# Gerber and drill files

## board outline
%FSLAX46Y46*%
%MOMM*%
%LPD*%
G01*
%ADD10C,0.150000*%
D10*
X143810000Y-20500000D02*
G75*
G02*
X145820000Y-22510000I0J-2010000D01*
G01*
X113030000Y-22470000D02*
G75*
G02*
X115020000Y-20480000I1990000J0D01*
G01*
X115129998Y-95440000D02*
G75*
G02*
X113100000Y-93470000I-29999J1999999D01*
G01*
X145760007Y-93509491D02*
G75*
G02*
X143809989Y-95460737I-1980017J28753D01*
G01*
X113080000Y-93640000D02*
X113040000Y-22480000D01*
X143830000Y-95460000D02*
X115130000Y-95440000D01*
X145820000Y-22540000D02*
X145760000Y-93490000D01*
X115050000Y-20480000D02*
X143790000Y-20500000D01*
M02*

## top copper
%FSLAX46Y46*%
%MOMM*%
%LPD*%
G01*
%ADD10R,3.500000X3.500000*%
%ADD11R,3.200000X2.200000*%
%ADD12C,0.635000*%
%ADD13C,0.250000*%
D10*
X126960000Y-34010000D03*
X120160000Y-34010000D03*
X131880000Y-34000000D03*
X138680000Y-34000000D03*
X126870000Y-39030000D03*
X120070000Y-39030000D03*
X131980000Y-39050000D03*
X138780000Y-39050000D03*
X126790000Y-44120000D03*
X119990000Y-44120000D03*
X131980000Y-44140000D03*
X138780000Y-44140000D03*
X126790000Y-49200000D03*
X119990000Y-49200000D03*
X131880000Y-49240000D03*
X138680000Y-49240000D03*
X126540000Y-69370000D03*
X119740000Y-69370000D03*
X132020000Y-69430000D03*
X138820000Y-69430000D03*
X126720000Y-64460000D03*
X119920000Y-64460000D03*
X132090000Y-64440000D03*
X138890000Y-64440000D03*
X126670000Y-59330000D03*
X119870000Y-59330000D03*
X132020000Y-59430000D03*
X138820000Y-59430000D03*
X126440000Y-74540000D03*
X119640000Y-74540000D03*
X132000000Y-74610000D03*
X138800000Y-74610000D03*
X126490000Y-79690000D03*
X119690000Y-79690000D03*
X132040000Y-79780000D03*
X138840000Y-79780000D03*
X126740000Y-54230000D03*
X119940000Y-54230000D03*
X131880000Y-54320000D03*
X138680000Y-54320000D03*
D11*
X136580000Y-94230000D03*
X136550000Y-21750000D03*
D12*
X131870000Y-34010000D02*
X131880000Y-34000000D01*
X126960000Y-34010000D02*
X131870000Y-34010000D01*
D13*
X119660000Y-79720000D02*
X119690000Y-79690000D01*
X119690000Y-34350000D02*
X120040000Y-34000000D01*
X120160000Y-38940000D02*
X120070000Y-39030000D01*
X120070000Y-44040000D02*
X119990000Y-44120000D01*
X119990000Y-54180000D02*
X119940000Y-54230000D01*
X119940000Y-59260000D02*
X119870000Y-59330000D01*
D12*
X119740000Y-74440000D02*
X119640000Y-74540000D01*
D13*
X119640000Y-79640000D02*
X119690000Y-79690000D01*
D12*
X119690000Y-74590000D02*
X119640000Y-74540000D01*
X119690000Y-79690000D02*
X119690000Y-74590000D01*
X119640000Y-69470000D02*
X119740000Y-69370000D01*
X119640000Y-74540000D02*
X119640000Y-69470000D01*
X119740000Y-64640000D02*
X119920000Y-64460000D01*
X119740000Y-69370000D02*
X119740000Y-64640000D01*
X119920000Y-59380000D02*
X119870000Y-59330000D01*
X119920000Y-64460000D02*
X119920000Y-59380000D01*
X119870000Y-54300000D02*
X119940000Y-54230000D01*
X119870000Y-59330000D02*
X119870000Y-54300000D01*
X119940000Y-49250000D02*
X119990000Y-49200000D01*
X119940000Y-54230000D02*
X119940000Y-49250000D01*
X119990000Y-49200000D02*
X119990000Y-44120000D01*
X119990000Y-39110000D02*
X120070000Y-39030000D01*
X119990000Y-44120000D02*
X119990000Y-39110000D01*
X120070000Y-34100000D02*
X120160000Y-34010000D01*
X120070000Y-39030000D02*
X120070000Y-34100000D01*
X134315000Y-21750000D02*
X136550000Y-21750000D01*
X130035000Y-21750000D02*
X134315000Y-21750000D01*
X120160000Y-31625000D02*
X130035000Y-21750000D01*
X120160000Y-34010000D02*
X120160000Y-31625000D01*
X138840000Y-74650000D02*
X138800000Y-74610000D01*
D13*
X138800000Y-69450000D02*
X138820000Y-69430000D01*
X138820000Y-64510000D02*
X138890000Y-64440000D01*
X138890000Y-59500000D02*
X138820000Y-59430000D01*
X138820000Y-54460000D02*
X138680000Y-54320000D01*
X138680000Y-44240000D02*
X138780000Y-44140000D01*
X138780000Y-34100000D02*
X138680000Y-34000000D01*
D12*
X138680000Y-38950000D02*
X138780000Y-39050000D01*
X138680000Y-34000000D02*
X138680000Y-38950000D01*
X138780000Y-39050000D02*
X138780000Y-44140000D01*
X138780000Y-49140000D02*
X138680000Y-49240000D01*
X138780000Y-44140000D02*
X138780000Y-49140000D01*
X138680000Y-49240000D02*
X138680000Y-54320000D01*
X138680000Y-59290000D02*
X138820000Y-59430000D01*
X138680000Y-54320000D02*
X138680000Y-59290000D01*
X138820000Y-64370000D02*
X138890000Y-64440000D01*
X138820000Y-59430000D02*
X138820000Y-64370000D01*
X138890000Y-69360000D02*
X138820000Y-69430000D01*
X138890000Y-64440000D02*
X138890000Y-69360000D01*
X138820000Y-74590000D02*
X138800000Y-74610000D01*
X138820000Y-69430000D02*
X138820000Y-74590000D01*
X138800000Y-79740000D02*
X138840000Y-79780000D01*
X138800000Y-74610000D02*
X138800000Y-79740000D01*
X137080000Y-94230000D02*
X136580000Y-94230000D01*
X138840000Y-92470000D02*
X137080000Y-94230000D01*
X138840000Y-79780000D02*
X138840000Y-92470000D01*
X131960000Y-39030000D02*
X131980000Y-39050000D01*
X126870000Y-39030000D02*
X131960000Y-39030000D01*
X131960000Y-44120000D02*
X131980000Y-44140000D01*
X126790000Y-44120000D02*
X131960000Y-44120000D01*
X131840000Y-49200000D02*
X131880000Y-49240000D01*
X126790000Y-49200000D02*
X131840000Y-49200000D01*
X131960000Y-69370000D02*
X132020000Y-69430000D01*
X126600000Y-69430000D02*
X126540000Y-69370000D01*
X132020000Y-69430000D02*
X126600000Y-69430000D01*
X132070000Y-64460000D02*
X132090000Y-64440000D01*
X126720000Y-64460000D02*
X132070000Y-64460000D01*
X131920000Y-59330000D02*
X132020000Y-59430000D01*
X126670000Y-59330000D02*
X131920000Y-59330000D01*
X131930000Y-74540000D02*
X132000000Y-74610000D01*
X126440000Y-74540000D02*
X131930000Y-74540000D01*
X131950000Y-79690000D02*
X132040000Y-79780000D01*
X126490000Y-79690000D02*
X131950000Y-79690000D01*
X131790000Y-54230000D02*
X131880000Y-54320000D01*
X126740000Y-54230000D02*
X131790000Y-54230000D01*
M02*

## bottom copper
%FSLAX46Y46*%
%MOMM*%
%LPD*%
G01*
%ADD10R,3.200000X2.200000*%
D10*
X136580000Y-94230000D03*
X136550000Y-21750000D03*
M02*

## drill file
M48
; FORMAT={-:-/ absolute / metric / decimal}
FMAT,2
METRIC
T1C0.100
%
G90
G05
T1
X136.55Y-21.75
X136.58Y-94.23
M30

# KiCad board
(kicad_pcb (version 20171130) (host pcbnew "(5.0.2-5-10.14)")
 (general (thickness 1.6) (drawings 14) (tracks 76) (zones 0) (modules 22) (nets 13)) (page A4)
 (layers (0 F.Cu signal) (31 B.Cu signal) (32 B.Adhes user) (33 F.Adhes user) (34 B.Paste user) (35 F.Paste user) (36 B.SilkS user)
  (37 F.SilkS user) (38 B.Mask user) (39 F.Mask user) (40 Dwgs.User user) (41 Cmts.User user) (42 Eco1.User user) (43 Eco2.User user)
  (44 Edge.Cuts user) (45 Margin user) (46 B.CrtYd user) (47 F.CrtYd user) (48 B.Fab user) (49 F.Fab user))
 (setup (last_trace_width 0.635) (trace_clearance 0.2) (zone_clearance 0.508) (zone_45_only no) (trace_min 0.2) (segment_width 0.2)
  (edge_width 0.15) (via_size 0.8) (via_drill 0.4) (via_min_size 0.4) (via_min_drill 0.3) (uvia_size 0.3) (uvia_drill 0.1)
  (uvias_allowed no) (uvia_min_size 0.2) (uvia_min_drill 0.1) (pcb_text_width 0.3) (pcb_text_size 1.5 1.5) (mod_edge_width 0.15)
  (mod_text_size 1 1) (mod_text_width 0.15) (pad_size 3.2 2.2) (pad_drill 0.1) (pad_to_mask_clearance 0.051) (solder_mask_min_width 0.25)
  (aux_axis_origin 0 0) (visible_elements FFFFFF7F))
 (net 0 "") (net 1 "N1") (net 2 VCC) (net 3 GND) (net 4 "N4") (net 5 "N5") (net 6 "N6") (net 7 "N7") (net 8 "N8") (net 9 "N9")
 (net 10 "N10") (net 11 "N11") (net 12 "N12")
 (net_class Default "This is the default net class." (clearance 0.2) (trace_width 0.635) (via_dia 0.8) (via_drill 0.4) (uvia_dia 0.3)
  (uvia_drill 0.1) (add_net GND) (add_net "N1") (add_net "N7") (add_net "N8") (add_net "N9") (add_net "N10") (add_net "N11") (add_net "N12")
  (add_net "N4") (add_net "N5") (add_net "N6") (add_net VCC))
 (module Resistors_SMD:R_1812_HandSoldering (layer F.Cu) (at 123.56 34.01)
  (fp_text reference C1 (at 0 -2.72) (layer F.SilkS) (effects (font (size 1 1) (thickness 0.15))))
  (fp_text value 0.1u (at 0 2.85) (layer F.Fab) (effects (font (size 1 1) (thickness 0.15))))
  (pad 2 smd rect (at 3.4 0) (size 3.5 3.5) (layers F.Cu F.Paste F.Mask) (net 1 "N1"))
  (pad 1 smd rect (at -3.4 0) (size 3.5 3.5) (layers F.Cu F.Paste F.Mask) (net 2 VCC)))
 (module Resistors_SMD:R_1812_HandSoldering (layer F.Cu) (at 135.28 34)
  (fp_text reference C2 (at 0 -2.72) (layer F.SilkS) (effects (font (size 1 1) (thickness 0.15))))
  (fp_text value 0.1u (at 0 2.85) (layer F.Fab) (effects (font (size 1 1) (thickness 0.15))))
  (pad 1 smd rect (at -3.4 0) (size 3.5 3.5) (layers F.Cu F.Paste F.Mask) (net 1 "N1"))
  (pad 2 smd rect (at 3.4 0) (size 3.5 3.5) (layers F.Cu F.Paste F.Mask) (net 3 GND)))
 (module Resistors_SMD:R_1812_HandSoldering (layer F.Cu) (at 123.47 39.03)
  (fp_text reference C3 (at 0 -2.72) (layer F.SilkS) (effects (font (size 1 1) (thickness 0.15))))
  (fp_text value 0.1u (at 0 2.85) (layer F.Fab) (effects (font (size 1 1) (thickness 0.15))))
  (pad 2 smd rect (at 3.4 0) (size 3.5 3.5) (layers F.Cu F.Paste F.Mask) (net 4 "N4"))
  (pad 1 smd rect (at -3.4 0) (size 3.5 3.5) (layers F.Cu F.Paste F.Mask) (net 2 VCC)))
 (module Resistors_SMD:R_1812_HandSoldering (layer F.Cu) (at 135.38 39.05)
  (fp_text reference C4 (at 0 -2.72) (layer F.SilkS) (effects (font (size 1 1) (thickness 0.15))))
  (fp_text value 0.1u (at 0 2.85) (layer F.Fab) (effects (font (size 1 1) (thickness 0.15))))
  (pad 1 smd rect (at -3.4 0) (size 3.5 3.5) (layers F.Cu F.Paste F.Mask) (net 4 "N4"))
  (pad 2 smd rect (at 3.4 0) (size 3.5 3.5) (layers F.Cu F.Paste F.Mask) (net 3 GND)))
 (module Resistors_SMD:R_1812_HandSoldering (layer F.Cu) (at 123.39 44.12)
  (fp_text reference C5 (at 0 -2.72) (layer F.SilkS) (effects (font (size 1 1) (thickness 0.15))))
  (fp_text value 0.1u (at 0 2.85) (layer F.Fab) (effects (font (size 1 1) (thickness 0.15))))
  (pad 2 smd rect (at 3.4 0) (size 3.5 3.5) (layers F.Cu F.Paste F.Mask) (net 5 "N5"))
  (pad 1 smd rect (at -3.4 0) (size 3.5 3.5) (layers F.Cu F.Paste F.Mask) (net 2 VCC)))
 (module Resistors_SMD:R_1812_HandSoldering (layer F.Cu) (at 135.38 44.14)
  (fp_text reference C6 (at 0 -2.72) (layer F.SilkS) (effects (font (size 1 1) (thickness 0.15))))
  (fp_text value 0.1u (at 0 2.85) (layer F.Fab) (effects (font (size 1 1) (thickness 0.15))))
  (pad 1 smd rect (at -3.4 0) (size 3.5 3.5) (layers F.Cu F.Paste F.Mask) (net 5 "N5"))
  (pad 2 smd rect (at 3.4 0) (size 3.5 3.5) (layers F.Cu F.Paste F.Mask) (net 3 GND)))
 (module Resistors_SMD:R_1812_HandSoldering (layer F.Cu) (at 123.39 49.2)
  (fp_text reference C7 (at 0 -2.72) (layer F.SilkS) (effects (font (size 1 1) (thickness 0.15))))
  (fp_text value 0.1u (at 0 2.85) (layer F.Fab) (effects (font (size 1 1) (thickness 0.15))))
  (pad 2 smd rect (at 3.4 0) (size 3.5 3.5) (layers F.Cu F.Paste F.Mask) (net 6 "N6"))
  (pad 1 smd rect (at -3.4 0) (size 3.5 3.5) (layers F.Cu F.Paste F.Mask) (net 2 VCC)))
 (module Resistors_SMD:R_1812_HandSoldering (layer F.Cu) (at 135.28 49.24)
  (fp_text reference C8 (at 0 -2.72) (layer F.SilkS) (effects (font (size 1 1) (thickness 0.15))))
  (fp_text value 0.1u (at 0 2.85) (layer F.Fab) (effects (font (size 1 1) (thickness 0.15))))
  (pad 1 smd rect (at -3.4 0) (size 3.5 3.5) (layers F.Cu F.Paste F.Mask) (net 6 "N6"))
  (pad 2 smd rect (at 3.4 0) (size 3.5 3.5) (layers F.Cu F.Paste F.Mask) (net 3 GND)))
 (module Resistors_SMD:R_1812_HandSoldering (layer F.Cu) (at 123.14 69.37)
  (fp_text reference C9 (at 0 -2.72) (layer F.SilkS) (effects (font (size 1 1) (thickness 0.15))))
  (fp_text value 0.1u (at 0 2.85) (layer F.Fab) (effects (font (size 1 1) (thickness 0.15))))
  (pad 2 smd rect (at 3.4 0) (size 3.5 3.5) (layers F.Cu F.Paste F.Mask) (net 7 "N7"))
  (pad 1 smd rect (at -3.4 0) (size 3.5 3.5) (layers F.Cu F.Paste F.Mask) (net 2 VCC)))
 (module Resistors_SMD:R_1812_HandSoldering (layer F.Cu) (at 135.42 69.43)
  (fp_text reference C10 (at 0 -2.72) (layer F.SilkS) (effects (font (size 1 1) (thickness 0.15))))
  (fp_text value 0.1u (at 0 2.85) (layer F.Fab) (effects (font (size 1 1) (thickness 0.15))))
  (pad 1 smd rect (at -3.4 0) (size 3.5 3.5) (layers F.Cu F.Paste F.Mask) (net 7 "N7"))
  (pad 2 smd rect (at 3.4 0) (size 3.5 3.5) (layers F.Cu F.Paste F.Mask) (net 3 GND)))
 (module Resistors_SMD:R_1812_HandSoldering (layer F.Cu) (at 123.32 64.46)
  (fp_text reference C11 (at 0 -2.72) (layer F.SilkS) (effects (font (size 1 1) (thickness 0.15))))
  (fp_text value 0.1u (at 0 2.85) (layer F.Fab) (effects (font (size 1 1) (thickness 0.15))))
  (pad 2 smd rect (at 3.4 0) (size 3.5 3.5) (layers F.Cu F.Paste F.Mask) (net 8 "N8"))
  (pad 1 smd rect (at -3.4 0) (size 3.5 3.5) (layers F.Cu F.Paste F.Mask) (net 2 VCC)))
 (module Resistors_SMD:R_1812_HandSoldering (layer F.Cu) (at 135.49 64.44)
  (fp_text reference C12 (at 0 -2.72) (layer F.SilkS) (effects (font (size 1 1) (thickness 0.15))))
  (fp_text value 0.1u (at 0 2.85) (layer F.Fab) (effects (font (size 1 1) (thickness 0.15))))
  (pad 1 smd rect (at -3.4 0) (size 3.5 3.5) (layers F.Cu F.Paste F.Mask) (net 8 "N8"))
  (pad 2 smd rect (at 3.4 0) (size 3.5 3.5) (layers F.Cu F.Paste F.Mask) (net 3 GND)))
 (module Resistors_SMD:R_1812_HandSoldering (layer F.Cu) (at 123.27 59.33)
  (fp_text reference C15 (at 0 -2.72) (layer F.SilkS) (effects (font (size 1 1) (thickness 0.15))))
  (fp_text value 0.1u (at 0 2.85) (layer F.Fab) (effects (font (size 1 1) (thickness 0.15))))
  (pad 2 smd rect (at 3.4 0) (size 3.5 3.5) (layers F.Cu F.Paste F.Mask) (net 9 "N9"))
  (pad 1 smd rect (at -3.4 0) (size 3.5 3.5) (layers F.Cu F.Paste F.Mask) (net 2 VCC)))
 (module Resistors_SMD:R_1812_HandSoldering (layer F.Cu) (at 135.42 59.43)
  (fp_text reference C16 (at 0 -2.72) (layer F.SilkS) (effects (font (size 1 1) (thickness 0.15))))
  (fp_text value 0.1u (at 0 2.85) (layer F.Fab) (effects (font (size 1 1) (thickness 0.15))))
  (pad 1 smd rect (at -3.4 0) (size 3.5 3.5) (layers F.Cu F.Paste F.Mask) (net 9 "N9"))
  (pad 2 smd rect (at 3.4 0) (size 3.5 3.5) (layers F.Cu F.Paste F.Mask) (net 3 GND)))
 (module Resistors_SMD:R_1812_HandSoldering (layer F.Cu) (at 123.04 74.54)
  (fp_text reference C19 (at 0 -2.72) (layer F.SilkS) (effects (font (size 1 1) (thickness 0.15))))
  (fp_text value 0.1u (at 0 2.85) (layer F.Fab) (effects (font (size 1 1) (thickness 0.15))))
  (pad 2 smd rect (at 3.4 0) (size 3.5 3.5) (layers F.Cu F.Paste F.Mask) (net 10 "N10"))
  (pad 1 smd rect (at -3.4 0) (size 3.5 3.5) (layers F.Cu F.Paste F.Mask) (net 2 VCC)))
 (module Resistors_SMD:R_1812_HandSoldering (layer F.Cu) (at 135.4 74.61)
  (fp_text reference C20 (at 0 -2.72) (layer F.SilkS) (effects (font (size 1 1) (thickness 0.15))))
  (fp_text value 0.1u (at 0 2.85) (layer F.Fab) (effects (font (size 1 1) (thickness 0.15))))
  (pad 1 smd rect (at -3.4 0) (size 3.5 3.5) (layers F.Cu F.Paste F.Mask) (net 10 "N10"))
  (pad 2 smd rect (at 3.4 0) (size 3.5 3.5) (layers F.Cu F.Paste F.Mask) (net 3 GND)))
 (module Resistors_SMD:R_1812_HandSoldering (layer F.Cu) (at 123.09 79.69)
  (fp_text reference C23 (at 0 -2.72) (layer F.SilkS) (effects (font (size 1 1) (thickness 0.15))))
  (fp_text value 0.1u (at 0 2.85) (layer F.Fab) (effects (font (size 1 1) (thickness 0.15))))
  (pad 2 smd rect (at 3.4 0) (size 3.5 3.5) (layers F.Cu F.Paste F.Mask) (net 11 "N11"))
  (pad 1 smd rect (at -3.4 0) (size 3.5 3.5) (layers F.Cu F.Paste F.Mask) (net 2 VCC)))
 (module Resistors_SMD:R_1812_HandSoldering (layer F.Cu) (at 135.44 79.78)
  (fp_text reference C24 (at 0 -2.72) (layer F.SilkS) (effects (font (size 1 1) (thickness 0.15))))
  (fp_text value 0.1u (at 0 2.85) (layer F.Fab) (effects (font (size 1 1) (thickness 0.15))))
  (pad 1 smd rect (at -3.4 0) (size 3.5 3.5) (layers F.Cu F.Paste F.Mask) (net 11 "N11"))
  (pad 2 smd rect (at 3.4 0) (size 3.5 3.5) (layers F.Cu F.Paste F.Mask) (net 3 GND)))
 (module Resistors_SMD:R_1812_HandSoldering (layer F.Cu) (at 123.34 54.23)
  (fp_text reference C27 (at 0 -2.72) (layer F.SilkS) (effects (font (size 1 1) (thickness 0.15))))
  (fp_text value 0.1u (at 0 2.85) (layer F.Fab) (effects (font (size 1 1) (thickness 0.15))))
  (pad 2 smd rect (at 3.4 0) (size 3.5 3.5) (layers F.Cu F.Paste F.Mask) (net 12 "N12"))
  (pad 1 smd rect (at -3.4 0) (size 3.5 3.5) (layers F.Cu F.Paste F.Mask) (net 2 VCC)))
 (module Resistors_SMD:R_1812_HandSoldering (layer F.Cu) (at 135.28 54.32)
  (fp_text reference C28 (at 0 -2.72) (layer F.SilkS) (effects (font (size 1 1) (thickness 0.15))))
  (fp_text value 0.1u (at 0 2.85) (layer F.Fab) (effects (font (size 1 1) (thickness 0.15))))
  (pad 1 smd rect (at -3.4 0) (size 3.5 3.5) (layers F.Cu F.Paste F.Mask) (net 12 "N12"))
  (pad 2 smd rect (at 3.4 0) (size 3.5 3.5) (layers F.Cu F.Paste F.Mask) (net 3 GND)))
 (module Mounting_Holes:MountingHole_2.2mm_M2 (layer F.Cu) (at 136.58 94.23)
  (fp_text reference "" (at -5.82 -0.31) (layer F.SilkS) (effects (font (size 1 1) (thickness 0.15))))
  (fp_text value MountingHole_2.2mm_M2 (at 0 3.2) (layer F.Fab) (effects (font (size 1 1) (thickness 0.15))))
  (pad "" thru_hole rect (at 0 0) (size 3.2 2.2) (drill 0.1) (layers *.Cu *.Mask) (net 3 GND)))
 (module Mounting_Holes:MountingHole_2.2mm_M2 (layer F.Cu) (at 136.55 21.75)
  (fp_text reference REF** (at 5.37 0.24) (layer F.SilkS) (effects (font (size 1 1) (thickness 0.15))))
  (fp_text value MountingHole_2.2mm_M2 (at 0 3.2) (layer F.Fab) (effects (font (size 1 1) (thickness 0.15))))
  (pad "" thru_hole rect (at 0 0) (size 3.2 2.2) (drill 0.1) (layers *.Cu *.Mask) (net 2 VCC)))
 (gr_arc (start 143.81 22.51) (end 145.82 22.51) (angle -90) (layer Edge.Cuts) (width 0.15))
 (gr_arc (start 115.02 22.47) (end 115.02 20.48) (angle -90) (layer Edge.Cuts) (width 0.15))
 (gr_arc (start 115.099999 93.440001) (end 113.1 93.47) (angle -90) (layer Edge.Cuts) (width 0.15))
 (gr_arc (start 143.77999 93.480738) (end 143.809989 95.460737) (angle -88.3) (layer Edge.Cuts) (width 0.15))
 (gr_line (start 113.08 93.64) (end 113.04 22.48) (layer Edge.Cuts) (width 0.15))
 (gr_line (start 143.83 95.46) (end 115.13 95.44) (layer Edge.Cuts) (width 0.15))
 (gr_line (start 145.82 22.54) (end 145.76 93.49) (layer Edge.Cuts) (width 0.15))
 (gr_line (start 115.05 20.48) (end 143.79 20.5) (layer Edge.Cuts) (width 0.15))
 (segment (start 131.87 34.01) (end 131.88 34) (width 0.635) (layer F.Cu) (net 1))
 (segment (start 126.96 34.01) (end 131.87 34.01) (width 0.635) (layer F.Cu) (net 1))
 (segment (start 119.66 79.72) (end 119.69 79.69) (width 0.25) (layer F.Cu) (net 2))
 (segment (start 119.69 34.35) (end 120.04 34) (width 0.25) (layer F.Cu) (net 2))
 (segment (start 120.16 38.94) (end 120.07 39.03) (width 0.25) (layer F.Cu) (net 2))
 (segment (start 120.07 44.04) (end 119.99 44.12) (width 0.25) (layer F.Cu) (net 2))
 (segment (start 119.99 54.18) (end 119.94 54.23) (width 0.25) (layer F.Cu) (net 2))
 (segment (start 119.94 59.26) (end 119.87 59.33) (width 0.25) (layer F.Cu) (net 2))
 (segment (start 119.74 74.44) (end 119.64 74.54) (width 0.635) (layer F.Cu) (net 2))
 (segment (start 119.64 79.64) (end 119.69 79.69) (width 0.25) (layer F.Cu) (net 2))
 (segment (start 119.69 74.59) (end 119.64 74.54) (width 0.635) (layer F.Cu) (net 2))
 (segment (start 119.69 79.69) (end 119.69 74.59) (width 0.635) (layer F.Cu) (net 2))
 (segment (start 119.64 69.47) (end 119.74 69.37) (width 0.635) (layer F.Cu) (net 2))
 (segment (start 119.64 74.54) (end 119.64 69.47) (width 0.635) (layer F.Cu) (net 2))
 (segment (start 119.74 64.64) (end 119.92 64.46) (width 0.635) (layer F.Cu) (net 2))
 (segment (start 119.74 69.37) (end 119.74 64.64) (width 0.635) (layer F.Cu) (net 2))
 (segment (start 119.92 59.38) (end 119.87 59.33) (width 0.635) (layer F.Cu) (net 2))
 (segment (start 119.92 64.46) (end 119.92 59.38) (width 0.635) (layer F.Cu) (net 2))
 (segment (start 119.87 54.3) (end 119.94 54.23) (width 0.635) (layer F.Cu) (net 2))
 (segment (start 119.87 59.33) (end 119.87 54.3) (width 0.635) (layer F.Cu) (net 2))
 (segment (start 119.94 49.25) (end 119.99 49.2) (width 0.635) (layer F.Cu) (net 2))
 (segment (start 119.94 54.23) (end 119.94 49.25) (width 0.635) (layer F.Cu) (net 2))
 (segment (start 119.99 49.2) (end 119.99 44.12) (width 0.635) (layer F.Cu) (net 2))
 (segment (start 119.99 39.11) (end 120.07 39.03) (width 0.635) (layer F.Cu) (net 2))
 (segment (start 119.99 44.12) (end 119.99 39.11) (width 0.635) (layer F.Cu) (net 2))
 (segment (start 120.07 34.1) (end 120.16 34.01) (width 0.635) (layer F.Cu) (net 2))
 (segment (start 120.07 39.03) (end 120.07 34.1) (width 0.635) (layer F.Cu) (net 2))
 (segment (start 134.315 21.75) (end 136.55 21.75) (width 0.635) (layer F.Cu) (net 2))
 (segment (start 130.035 21.75) (end 134.315 21.75) (width 0.635) (layer F.Cu) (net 2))
 (segment (start 120.16 31.625) (end 130.035 21.75) (width 0.635) (layer F.Cu) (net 2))
 (segment (start 120.16 34.01) (end 120.16 31.625) (width 0.635) (layer F.Cu) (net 2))
 (segment (start 138.84 74.65) (end 138.8 74.61) (width 0.635) (layer F.Cu) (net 3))
 (segment (start 138.8 69.45) (end 138.82 69.43) (width 0.25) (layer F.Cu) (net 3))
 (segment (start 138.82 64.51) (end 138.89 64.44) (width 0.25) (layer F.Cu) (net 3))
 (segment (start 138.89 59.5) (end 138.82 59.43) (width 0.25) (layer F.Cu) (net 3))
 (segment (start 138.82 54.46) (end 138.68 54.32) (width 0.25) (layer F.Cu) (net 3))
 (segment (start 138.68 44.24) (end 138.78 44.14) (width 0.25) (layer F.Cu) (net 3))
 (segment (start 138.78 34.1) (end 138.68 34) (width 0.25) (layer F.Cu) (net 3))
 (segment (start 138.68 38.95) (end 138.78 39.05) (width 0.635) (layer F.Cu) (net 3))
 (segment (start 138.68 34) (end 138.68 38.95) (width 0.635) (layer F.Cu) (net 3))
 (segment (start 138.78 39.05) (end 138.78 44.14) (width 0.635) (layer F.Cu) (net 3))
 (segment (start 138.78 49.14) (end 138.68 49.24) (width 0.635) (layer F.Cu) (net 3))
 (segment (start 138.78 44.14) (end 138.78 49.14) (width 0.635) (layer F.Cu) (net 3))
 (segment (start 138.68 49.24) (end 138.68 54.32) (width 0.635) (layer F.Cu) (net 3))
 (segment (start 138.68 59.29) (end 138.82 59.43) (width 0.635) (layer F.Cu) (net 3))
 (segment (start 138.68 54.32) (end 138.68 59.29) (width 0.635) (layer F.Cu) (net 3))
 (segment (start 138.82 64.37) (end 138.89 64.44) (width 0.635) (layer F.Cu) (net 3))
 (segment (start 138.82 59.43) (end 138.82 64.37) (width 0.635) (layer F.Cu) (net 3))
 (segment (start 138.89 69.36) (end 138.82 69.43) (width 0.635) (layer F.Cu) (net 3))
 (segment (start 138.89 64.44) (end 138.89 69.36) (width 0.635) (layer F.Cu) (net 3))
 (segment (start 138.82 74.59) (end 138.8 74.61) (width 0.635) (layer F.Cu) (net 3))
 (segment (start 138.82 69.43) (end 138.82 74.59) (width 0.635) (layer F.Cu) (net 3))
 (segment (start 138.8 79.74) (end 138.84 79.78) (width 0.635) (layer F.Cu) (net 3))
 (segment (start 138.8 74.61) (end 138.8 79.74) (width 0.635) (layer F.Cu) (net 3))
 (segment (start 137.08 94.23) (end 136.58 94.23) (width 0.635) (layer F.Cu) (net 3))
 (segment (start 138.84 92.47) (end 137.08 94.23) (width 0.635) (layer F.Cu) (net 3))
 (segment (start 138.84 79.78) (end 138.84 92.47) (width 0.635) (layer F.Cu) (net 3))
 (segment (start 131.96 39.03) (end 131.98 39.05) (width 0.635) (layer F.Cu) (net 4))
 (segment (start 126.87 39.03) (end 131.96 39.03) (width 0.635) (layer F.Cu) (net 4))
 (segment (start 131.96 44.12) (end 131.98 44.14) (width 0.635) (layer F.Cu) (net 5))
 (segment (start 126.79 44.12) (end 131.96 44.12) (width 0.635) (layer F.Cu) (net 5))
 (segment (start 131.84 49.2) (end 131.88 49.24) (width 0.635) (layer F.Cu) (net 6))
 (segment (start 126.79 49.2) (end 131.84 49.2) (width 0.635) (layer F.Cu) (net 6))
 (segment (start 131.96 69.37) (end 132.02 69.43) (width 0.635) (layer F.Cu) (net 7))
 (segment (start 126.6 69.43) (end 126.54 69.37) (width 0.635) (layer F.Cu) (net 7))
 (segment (start 132.02 69.43) (end 126.6 69.43) (width 0.635) (layer F.Cu) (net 7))
 (segment (start 132.07 64.46) (end 132.09 64.44) (width 0.635) (layer F.Cu) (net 8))
 (segment (start 126.72 64.46) (end 132.07 64.46) (width 0.635) (layer F.Cu) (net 8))
 (segment (start 131.92 59.33) (end 132.02 59.43) (width 0.635) (layer F.Cu) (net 9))
 (segment (start 126.67 59.33) (end 131.92 59.33) (width 0.635) (layer F.Cu) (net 9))
 (segment (start 131.93 74.54) (end 132 74.61) (width 0.635) (layer F.Cu) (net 10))
 (segment (start 126.44 74.54) (end 131.93 74.54) (width 0.635) (layer F.Cu) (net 10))
 (segment (start 131.95 79.69) (end 132.04 79.78) (width 0.635) (layer F.Cu) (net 11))
 (segment (start 126.49 79.69) (end 131.95 79.69) (width 0.635) (layer F.Cu) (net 11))
 (segment (start 131.79 54.23) (end 131.88 54.32) (width 0.635) (layer F.Cu) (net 12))
 (segment (start 126.74 54.23) (end 131.79 54.23) (width 0.635) (layer F.Cu) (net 12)))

